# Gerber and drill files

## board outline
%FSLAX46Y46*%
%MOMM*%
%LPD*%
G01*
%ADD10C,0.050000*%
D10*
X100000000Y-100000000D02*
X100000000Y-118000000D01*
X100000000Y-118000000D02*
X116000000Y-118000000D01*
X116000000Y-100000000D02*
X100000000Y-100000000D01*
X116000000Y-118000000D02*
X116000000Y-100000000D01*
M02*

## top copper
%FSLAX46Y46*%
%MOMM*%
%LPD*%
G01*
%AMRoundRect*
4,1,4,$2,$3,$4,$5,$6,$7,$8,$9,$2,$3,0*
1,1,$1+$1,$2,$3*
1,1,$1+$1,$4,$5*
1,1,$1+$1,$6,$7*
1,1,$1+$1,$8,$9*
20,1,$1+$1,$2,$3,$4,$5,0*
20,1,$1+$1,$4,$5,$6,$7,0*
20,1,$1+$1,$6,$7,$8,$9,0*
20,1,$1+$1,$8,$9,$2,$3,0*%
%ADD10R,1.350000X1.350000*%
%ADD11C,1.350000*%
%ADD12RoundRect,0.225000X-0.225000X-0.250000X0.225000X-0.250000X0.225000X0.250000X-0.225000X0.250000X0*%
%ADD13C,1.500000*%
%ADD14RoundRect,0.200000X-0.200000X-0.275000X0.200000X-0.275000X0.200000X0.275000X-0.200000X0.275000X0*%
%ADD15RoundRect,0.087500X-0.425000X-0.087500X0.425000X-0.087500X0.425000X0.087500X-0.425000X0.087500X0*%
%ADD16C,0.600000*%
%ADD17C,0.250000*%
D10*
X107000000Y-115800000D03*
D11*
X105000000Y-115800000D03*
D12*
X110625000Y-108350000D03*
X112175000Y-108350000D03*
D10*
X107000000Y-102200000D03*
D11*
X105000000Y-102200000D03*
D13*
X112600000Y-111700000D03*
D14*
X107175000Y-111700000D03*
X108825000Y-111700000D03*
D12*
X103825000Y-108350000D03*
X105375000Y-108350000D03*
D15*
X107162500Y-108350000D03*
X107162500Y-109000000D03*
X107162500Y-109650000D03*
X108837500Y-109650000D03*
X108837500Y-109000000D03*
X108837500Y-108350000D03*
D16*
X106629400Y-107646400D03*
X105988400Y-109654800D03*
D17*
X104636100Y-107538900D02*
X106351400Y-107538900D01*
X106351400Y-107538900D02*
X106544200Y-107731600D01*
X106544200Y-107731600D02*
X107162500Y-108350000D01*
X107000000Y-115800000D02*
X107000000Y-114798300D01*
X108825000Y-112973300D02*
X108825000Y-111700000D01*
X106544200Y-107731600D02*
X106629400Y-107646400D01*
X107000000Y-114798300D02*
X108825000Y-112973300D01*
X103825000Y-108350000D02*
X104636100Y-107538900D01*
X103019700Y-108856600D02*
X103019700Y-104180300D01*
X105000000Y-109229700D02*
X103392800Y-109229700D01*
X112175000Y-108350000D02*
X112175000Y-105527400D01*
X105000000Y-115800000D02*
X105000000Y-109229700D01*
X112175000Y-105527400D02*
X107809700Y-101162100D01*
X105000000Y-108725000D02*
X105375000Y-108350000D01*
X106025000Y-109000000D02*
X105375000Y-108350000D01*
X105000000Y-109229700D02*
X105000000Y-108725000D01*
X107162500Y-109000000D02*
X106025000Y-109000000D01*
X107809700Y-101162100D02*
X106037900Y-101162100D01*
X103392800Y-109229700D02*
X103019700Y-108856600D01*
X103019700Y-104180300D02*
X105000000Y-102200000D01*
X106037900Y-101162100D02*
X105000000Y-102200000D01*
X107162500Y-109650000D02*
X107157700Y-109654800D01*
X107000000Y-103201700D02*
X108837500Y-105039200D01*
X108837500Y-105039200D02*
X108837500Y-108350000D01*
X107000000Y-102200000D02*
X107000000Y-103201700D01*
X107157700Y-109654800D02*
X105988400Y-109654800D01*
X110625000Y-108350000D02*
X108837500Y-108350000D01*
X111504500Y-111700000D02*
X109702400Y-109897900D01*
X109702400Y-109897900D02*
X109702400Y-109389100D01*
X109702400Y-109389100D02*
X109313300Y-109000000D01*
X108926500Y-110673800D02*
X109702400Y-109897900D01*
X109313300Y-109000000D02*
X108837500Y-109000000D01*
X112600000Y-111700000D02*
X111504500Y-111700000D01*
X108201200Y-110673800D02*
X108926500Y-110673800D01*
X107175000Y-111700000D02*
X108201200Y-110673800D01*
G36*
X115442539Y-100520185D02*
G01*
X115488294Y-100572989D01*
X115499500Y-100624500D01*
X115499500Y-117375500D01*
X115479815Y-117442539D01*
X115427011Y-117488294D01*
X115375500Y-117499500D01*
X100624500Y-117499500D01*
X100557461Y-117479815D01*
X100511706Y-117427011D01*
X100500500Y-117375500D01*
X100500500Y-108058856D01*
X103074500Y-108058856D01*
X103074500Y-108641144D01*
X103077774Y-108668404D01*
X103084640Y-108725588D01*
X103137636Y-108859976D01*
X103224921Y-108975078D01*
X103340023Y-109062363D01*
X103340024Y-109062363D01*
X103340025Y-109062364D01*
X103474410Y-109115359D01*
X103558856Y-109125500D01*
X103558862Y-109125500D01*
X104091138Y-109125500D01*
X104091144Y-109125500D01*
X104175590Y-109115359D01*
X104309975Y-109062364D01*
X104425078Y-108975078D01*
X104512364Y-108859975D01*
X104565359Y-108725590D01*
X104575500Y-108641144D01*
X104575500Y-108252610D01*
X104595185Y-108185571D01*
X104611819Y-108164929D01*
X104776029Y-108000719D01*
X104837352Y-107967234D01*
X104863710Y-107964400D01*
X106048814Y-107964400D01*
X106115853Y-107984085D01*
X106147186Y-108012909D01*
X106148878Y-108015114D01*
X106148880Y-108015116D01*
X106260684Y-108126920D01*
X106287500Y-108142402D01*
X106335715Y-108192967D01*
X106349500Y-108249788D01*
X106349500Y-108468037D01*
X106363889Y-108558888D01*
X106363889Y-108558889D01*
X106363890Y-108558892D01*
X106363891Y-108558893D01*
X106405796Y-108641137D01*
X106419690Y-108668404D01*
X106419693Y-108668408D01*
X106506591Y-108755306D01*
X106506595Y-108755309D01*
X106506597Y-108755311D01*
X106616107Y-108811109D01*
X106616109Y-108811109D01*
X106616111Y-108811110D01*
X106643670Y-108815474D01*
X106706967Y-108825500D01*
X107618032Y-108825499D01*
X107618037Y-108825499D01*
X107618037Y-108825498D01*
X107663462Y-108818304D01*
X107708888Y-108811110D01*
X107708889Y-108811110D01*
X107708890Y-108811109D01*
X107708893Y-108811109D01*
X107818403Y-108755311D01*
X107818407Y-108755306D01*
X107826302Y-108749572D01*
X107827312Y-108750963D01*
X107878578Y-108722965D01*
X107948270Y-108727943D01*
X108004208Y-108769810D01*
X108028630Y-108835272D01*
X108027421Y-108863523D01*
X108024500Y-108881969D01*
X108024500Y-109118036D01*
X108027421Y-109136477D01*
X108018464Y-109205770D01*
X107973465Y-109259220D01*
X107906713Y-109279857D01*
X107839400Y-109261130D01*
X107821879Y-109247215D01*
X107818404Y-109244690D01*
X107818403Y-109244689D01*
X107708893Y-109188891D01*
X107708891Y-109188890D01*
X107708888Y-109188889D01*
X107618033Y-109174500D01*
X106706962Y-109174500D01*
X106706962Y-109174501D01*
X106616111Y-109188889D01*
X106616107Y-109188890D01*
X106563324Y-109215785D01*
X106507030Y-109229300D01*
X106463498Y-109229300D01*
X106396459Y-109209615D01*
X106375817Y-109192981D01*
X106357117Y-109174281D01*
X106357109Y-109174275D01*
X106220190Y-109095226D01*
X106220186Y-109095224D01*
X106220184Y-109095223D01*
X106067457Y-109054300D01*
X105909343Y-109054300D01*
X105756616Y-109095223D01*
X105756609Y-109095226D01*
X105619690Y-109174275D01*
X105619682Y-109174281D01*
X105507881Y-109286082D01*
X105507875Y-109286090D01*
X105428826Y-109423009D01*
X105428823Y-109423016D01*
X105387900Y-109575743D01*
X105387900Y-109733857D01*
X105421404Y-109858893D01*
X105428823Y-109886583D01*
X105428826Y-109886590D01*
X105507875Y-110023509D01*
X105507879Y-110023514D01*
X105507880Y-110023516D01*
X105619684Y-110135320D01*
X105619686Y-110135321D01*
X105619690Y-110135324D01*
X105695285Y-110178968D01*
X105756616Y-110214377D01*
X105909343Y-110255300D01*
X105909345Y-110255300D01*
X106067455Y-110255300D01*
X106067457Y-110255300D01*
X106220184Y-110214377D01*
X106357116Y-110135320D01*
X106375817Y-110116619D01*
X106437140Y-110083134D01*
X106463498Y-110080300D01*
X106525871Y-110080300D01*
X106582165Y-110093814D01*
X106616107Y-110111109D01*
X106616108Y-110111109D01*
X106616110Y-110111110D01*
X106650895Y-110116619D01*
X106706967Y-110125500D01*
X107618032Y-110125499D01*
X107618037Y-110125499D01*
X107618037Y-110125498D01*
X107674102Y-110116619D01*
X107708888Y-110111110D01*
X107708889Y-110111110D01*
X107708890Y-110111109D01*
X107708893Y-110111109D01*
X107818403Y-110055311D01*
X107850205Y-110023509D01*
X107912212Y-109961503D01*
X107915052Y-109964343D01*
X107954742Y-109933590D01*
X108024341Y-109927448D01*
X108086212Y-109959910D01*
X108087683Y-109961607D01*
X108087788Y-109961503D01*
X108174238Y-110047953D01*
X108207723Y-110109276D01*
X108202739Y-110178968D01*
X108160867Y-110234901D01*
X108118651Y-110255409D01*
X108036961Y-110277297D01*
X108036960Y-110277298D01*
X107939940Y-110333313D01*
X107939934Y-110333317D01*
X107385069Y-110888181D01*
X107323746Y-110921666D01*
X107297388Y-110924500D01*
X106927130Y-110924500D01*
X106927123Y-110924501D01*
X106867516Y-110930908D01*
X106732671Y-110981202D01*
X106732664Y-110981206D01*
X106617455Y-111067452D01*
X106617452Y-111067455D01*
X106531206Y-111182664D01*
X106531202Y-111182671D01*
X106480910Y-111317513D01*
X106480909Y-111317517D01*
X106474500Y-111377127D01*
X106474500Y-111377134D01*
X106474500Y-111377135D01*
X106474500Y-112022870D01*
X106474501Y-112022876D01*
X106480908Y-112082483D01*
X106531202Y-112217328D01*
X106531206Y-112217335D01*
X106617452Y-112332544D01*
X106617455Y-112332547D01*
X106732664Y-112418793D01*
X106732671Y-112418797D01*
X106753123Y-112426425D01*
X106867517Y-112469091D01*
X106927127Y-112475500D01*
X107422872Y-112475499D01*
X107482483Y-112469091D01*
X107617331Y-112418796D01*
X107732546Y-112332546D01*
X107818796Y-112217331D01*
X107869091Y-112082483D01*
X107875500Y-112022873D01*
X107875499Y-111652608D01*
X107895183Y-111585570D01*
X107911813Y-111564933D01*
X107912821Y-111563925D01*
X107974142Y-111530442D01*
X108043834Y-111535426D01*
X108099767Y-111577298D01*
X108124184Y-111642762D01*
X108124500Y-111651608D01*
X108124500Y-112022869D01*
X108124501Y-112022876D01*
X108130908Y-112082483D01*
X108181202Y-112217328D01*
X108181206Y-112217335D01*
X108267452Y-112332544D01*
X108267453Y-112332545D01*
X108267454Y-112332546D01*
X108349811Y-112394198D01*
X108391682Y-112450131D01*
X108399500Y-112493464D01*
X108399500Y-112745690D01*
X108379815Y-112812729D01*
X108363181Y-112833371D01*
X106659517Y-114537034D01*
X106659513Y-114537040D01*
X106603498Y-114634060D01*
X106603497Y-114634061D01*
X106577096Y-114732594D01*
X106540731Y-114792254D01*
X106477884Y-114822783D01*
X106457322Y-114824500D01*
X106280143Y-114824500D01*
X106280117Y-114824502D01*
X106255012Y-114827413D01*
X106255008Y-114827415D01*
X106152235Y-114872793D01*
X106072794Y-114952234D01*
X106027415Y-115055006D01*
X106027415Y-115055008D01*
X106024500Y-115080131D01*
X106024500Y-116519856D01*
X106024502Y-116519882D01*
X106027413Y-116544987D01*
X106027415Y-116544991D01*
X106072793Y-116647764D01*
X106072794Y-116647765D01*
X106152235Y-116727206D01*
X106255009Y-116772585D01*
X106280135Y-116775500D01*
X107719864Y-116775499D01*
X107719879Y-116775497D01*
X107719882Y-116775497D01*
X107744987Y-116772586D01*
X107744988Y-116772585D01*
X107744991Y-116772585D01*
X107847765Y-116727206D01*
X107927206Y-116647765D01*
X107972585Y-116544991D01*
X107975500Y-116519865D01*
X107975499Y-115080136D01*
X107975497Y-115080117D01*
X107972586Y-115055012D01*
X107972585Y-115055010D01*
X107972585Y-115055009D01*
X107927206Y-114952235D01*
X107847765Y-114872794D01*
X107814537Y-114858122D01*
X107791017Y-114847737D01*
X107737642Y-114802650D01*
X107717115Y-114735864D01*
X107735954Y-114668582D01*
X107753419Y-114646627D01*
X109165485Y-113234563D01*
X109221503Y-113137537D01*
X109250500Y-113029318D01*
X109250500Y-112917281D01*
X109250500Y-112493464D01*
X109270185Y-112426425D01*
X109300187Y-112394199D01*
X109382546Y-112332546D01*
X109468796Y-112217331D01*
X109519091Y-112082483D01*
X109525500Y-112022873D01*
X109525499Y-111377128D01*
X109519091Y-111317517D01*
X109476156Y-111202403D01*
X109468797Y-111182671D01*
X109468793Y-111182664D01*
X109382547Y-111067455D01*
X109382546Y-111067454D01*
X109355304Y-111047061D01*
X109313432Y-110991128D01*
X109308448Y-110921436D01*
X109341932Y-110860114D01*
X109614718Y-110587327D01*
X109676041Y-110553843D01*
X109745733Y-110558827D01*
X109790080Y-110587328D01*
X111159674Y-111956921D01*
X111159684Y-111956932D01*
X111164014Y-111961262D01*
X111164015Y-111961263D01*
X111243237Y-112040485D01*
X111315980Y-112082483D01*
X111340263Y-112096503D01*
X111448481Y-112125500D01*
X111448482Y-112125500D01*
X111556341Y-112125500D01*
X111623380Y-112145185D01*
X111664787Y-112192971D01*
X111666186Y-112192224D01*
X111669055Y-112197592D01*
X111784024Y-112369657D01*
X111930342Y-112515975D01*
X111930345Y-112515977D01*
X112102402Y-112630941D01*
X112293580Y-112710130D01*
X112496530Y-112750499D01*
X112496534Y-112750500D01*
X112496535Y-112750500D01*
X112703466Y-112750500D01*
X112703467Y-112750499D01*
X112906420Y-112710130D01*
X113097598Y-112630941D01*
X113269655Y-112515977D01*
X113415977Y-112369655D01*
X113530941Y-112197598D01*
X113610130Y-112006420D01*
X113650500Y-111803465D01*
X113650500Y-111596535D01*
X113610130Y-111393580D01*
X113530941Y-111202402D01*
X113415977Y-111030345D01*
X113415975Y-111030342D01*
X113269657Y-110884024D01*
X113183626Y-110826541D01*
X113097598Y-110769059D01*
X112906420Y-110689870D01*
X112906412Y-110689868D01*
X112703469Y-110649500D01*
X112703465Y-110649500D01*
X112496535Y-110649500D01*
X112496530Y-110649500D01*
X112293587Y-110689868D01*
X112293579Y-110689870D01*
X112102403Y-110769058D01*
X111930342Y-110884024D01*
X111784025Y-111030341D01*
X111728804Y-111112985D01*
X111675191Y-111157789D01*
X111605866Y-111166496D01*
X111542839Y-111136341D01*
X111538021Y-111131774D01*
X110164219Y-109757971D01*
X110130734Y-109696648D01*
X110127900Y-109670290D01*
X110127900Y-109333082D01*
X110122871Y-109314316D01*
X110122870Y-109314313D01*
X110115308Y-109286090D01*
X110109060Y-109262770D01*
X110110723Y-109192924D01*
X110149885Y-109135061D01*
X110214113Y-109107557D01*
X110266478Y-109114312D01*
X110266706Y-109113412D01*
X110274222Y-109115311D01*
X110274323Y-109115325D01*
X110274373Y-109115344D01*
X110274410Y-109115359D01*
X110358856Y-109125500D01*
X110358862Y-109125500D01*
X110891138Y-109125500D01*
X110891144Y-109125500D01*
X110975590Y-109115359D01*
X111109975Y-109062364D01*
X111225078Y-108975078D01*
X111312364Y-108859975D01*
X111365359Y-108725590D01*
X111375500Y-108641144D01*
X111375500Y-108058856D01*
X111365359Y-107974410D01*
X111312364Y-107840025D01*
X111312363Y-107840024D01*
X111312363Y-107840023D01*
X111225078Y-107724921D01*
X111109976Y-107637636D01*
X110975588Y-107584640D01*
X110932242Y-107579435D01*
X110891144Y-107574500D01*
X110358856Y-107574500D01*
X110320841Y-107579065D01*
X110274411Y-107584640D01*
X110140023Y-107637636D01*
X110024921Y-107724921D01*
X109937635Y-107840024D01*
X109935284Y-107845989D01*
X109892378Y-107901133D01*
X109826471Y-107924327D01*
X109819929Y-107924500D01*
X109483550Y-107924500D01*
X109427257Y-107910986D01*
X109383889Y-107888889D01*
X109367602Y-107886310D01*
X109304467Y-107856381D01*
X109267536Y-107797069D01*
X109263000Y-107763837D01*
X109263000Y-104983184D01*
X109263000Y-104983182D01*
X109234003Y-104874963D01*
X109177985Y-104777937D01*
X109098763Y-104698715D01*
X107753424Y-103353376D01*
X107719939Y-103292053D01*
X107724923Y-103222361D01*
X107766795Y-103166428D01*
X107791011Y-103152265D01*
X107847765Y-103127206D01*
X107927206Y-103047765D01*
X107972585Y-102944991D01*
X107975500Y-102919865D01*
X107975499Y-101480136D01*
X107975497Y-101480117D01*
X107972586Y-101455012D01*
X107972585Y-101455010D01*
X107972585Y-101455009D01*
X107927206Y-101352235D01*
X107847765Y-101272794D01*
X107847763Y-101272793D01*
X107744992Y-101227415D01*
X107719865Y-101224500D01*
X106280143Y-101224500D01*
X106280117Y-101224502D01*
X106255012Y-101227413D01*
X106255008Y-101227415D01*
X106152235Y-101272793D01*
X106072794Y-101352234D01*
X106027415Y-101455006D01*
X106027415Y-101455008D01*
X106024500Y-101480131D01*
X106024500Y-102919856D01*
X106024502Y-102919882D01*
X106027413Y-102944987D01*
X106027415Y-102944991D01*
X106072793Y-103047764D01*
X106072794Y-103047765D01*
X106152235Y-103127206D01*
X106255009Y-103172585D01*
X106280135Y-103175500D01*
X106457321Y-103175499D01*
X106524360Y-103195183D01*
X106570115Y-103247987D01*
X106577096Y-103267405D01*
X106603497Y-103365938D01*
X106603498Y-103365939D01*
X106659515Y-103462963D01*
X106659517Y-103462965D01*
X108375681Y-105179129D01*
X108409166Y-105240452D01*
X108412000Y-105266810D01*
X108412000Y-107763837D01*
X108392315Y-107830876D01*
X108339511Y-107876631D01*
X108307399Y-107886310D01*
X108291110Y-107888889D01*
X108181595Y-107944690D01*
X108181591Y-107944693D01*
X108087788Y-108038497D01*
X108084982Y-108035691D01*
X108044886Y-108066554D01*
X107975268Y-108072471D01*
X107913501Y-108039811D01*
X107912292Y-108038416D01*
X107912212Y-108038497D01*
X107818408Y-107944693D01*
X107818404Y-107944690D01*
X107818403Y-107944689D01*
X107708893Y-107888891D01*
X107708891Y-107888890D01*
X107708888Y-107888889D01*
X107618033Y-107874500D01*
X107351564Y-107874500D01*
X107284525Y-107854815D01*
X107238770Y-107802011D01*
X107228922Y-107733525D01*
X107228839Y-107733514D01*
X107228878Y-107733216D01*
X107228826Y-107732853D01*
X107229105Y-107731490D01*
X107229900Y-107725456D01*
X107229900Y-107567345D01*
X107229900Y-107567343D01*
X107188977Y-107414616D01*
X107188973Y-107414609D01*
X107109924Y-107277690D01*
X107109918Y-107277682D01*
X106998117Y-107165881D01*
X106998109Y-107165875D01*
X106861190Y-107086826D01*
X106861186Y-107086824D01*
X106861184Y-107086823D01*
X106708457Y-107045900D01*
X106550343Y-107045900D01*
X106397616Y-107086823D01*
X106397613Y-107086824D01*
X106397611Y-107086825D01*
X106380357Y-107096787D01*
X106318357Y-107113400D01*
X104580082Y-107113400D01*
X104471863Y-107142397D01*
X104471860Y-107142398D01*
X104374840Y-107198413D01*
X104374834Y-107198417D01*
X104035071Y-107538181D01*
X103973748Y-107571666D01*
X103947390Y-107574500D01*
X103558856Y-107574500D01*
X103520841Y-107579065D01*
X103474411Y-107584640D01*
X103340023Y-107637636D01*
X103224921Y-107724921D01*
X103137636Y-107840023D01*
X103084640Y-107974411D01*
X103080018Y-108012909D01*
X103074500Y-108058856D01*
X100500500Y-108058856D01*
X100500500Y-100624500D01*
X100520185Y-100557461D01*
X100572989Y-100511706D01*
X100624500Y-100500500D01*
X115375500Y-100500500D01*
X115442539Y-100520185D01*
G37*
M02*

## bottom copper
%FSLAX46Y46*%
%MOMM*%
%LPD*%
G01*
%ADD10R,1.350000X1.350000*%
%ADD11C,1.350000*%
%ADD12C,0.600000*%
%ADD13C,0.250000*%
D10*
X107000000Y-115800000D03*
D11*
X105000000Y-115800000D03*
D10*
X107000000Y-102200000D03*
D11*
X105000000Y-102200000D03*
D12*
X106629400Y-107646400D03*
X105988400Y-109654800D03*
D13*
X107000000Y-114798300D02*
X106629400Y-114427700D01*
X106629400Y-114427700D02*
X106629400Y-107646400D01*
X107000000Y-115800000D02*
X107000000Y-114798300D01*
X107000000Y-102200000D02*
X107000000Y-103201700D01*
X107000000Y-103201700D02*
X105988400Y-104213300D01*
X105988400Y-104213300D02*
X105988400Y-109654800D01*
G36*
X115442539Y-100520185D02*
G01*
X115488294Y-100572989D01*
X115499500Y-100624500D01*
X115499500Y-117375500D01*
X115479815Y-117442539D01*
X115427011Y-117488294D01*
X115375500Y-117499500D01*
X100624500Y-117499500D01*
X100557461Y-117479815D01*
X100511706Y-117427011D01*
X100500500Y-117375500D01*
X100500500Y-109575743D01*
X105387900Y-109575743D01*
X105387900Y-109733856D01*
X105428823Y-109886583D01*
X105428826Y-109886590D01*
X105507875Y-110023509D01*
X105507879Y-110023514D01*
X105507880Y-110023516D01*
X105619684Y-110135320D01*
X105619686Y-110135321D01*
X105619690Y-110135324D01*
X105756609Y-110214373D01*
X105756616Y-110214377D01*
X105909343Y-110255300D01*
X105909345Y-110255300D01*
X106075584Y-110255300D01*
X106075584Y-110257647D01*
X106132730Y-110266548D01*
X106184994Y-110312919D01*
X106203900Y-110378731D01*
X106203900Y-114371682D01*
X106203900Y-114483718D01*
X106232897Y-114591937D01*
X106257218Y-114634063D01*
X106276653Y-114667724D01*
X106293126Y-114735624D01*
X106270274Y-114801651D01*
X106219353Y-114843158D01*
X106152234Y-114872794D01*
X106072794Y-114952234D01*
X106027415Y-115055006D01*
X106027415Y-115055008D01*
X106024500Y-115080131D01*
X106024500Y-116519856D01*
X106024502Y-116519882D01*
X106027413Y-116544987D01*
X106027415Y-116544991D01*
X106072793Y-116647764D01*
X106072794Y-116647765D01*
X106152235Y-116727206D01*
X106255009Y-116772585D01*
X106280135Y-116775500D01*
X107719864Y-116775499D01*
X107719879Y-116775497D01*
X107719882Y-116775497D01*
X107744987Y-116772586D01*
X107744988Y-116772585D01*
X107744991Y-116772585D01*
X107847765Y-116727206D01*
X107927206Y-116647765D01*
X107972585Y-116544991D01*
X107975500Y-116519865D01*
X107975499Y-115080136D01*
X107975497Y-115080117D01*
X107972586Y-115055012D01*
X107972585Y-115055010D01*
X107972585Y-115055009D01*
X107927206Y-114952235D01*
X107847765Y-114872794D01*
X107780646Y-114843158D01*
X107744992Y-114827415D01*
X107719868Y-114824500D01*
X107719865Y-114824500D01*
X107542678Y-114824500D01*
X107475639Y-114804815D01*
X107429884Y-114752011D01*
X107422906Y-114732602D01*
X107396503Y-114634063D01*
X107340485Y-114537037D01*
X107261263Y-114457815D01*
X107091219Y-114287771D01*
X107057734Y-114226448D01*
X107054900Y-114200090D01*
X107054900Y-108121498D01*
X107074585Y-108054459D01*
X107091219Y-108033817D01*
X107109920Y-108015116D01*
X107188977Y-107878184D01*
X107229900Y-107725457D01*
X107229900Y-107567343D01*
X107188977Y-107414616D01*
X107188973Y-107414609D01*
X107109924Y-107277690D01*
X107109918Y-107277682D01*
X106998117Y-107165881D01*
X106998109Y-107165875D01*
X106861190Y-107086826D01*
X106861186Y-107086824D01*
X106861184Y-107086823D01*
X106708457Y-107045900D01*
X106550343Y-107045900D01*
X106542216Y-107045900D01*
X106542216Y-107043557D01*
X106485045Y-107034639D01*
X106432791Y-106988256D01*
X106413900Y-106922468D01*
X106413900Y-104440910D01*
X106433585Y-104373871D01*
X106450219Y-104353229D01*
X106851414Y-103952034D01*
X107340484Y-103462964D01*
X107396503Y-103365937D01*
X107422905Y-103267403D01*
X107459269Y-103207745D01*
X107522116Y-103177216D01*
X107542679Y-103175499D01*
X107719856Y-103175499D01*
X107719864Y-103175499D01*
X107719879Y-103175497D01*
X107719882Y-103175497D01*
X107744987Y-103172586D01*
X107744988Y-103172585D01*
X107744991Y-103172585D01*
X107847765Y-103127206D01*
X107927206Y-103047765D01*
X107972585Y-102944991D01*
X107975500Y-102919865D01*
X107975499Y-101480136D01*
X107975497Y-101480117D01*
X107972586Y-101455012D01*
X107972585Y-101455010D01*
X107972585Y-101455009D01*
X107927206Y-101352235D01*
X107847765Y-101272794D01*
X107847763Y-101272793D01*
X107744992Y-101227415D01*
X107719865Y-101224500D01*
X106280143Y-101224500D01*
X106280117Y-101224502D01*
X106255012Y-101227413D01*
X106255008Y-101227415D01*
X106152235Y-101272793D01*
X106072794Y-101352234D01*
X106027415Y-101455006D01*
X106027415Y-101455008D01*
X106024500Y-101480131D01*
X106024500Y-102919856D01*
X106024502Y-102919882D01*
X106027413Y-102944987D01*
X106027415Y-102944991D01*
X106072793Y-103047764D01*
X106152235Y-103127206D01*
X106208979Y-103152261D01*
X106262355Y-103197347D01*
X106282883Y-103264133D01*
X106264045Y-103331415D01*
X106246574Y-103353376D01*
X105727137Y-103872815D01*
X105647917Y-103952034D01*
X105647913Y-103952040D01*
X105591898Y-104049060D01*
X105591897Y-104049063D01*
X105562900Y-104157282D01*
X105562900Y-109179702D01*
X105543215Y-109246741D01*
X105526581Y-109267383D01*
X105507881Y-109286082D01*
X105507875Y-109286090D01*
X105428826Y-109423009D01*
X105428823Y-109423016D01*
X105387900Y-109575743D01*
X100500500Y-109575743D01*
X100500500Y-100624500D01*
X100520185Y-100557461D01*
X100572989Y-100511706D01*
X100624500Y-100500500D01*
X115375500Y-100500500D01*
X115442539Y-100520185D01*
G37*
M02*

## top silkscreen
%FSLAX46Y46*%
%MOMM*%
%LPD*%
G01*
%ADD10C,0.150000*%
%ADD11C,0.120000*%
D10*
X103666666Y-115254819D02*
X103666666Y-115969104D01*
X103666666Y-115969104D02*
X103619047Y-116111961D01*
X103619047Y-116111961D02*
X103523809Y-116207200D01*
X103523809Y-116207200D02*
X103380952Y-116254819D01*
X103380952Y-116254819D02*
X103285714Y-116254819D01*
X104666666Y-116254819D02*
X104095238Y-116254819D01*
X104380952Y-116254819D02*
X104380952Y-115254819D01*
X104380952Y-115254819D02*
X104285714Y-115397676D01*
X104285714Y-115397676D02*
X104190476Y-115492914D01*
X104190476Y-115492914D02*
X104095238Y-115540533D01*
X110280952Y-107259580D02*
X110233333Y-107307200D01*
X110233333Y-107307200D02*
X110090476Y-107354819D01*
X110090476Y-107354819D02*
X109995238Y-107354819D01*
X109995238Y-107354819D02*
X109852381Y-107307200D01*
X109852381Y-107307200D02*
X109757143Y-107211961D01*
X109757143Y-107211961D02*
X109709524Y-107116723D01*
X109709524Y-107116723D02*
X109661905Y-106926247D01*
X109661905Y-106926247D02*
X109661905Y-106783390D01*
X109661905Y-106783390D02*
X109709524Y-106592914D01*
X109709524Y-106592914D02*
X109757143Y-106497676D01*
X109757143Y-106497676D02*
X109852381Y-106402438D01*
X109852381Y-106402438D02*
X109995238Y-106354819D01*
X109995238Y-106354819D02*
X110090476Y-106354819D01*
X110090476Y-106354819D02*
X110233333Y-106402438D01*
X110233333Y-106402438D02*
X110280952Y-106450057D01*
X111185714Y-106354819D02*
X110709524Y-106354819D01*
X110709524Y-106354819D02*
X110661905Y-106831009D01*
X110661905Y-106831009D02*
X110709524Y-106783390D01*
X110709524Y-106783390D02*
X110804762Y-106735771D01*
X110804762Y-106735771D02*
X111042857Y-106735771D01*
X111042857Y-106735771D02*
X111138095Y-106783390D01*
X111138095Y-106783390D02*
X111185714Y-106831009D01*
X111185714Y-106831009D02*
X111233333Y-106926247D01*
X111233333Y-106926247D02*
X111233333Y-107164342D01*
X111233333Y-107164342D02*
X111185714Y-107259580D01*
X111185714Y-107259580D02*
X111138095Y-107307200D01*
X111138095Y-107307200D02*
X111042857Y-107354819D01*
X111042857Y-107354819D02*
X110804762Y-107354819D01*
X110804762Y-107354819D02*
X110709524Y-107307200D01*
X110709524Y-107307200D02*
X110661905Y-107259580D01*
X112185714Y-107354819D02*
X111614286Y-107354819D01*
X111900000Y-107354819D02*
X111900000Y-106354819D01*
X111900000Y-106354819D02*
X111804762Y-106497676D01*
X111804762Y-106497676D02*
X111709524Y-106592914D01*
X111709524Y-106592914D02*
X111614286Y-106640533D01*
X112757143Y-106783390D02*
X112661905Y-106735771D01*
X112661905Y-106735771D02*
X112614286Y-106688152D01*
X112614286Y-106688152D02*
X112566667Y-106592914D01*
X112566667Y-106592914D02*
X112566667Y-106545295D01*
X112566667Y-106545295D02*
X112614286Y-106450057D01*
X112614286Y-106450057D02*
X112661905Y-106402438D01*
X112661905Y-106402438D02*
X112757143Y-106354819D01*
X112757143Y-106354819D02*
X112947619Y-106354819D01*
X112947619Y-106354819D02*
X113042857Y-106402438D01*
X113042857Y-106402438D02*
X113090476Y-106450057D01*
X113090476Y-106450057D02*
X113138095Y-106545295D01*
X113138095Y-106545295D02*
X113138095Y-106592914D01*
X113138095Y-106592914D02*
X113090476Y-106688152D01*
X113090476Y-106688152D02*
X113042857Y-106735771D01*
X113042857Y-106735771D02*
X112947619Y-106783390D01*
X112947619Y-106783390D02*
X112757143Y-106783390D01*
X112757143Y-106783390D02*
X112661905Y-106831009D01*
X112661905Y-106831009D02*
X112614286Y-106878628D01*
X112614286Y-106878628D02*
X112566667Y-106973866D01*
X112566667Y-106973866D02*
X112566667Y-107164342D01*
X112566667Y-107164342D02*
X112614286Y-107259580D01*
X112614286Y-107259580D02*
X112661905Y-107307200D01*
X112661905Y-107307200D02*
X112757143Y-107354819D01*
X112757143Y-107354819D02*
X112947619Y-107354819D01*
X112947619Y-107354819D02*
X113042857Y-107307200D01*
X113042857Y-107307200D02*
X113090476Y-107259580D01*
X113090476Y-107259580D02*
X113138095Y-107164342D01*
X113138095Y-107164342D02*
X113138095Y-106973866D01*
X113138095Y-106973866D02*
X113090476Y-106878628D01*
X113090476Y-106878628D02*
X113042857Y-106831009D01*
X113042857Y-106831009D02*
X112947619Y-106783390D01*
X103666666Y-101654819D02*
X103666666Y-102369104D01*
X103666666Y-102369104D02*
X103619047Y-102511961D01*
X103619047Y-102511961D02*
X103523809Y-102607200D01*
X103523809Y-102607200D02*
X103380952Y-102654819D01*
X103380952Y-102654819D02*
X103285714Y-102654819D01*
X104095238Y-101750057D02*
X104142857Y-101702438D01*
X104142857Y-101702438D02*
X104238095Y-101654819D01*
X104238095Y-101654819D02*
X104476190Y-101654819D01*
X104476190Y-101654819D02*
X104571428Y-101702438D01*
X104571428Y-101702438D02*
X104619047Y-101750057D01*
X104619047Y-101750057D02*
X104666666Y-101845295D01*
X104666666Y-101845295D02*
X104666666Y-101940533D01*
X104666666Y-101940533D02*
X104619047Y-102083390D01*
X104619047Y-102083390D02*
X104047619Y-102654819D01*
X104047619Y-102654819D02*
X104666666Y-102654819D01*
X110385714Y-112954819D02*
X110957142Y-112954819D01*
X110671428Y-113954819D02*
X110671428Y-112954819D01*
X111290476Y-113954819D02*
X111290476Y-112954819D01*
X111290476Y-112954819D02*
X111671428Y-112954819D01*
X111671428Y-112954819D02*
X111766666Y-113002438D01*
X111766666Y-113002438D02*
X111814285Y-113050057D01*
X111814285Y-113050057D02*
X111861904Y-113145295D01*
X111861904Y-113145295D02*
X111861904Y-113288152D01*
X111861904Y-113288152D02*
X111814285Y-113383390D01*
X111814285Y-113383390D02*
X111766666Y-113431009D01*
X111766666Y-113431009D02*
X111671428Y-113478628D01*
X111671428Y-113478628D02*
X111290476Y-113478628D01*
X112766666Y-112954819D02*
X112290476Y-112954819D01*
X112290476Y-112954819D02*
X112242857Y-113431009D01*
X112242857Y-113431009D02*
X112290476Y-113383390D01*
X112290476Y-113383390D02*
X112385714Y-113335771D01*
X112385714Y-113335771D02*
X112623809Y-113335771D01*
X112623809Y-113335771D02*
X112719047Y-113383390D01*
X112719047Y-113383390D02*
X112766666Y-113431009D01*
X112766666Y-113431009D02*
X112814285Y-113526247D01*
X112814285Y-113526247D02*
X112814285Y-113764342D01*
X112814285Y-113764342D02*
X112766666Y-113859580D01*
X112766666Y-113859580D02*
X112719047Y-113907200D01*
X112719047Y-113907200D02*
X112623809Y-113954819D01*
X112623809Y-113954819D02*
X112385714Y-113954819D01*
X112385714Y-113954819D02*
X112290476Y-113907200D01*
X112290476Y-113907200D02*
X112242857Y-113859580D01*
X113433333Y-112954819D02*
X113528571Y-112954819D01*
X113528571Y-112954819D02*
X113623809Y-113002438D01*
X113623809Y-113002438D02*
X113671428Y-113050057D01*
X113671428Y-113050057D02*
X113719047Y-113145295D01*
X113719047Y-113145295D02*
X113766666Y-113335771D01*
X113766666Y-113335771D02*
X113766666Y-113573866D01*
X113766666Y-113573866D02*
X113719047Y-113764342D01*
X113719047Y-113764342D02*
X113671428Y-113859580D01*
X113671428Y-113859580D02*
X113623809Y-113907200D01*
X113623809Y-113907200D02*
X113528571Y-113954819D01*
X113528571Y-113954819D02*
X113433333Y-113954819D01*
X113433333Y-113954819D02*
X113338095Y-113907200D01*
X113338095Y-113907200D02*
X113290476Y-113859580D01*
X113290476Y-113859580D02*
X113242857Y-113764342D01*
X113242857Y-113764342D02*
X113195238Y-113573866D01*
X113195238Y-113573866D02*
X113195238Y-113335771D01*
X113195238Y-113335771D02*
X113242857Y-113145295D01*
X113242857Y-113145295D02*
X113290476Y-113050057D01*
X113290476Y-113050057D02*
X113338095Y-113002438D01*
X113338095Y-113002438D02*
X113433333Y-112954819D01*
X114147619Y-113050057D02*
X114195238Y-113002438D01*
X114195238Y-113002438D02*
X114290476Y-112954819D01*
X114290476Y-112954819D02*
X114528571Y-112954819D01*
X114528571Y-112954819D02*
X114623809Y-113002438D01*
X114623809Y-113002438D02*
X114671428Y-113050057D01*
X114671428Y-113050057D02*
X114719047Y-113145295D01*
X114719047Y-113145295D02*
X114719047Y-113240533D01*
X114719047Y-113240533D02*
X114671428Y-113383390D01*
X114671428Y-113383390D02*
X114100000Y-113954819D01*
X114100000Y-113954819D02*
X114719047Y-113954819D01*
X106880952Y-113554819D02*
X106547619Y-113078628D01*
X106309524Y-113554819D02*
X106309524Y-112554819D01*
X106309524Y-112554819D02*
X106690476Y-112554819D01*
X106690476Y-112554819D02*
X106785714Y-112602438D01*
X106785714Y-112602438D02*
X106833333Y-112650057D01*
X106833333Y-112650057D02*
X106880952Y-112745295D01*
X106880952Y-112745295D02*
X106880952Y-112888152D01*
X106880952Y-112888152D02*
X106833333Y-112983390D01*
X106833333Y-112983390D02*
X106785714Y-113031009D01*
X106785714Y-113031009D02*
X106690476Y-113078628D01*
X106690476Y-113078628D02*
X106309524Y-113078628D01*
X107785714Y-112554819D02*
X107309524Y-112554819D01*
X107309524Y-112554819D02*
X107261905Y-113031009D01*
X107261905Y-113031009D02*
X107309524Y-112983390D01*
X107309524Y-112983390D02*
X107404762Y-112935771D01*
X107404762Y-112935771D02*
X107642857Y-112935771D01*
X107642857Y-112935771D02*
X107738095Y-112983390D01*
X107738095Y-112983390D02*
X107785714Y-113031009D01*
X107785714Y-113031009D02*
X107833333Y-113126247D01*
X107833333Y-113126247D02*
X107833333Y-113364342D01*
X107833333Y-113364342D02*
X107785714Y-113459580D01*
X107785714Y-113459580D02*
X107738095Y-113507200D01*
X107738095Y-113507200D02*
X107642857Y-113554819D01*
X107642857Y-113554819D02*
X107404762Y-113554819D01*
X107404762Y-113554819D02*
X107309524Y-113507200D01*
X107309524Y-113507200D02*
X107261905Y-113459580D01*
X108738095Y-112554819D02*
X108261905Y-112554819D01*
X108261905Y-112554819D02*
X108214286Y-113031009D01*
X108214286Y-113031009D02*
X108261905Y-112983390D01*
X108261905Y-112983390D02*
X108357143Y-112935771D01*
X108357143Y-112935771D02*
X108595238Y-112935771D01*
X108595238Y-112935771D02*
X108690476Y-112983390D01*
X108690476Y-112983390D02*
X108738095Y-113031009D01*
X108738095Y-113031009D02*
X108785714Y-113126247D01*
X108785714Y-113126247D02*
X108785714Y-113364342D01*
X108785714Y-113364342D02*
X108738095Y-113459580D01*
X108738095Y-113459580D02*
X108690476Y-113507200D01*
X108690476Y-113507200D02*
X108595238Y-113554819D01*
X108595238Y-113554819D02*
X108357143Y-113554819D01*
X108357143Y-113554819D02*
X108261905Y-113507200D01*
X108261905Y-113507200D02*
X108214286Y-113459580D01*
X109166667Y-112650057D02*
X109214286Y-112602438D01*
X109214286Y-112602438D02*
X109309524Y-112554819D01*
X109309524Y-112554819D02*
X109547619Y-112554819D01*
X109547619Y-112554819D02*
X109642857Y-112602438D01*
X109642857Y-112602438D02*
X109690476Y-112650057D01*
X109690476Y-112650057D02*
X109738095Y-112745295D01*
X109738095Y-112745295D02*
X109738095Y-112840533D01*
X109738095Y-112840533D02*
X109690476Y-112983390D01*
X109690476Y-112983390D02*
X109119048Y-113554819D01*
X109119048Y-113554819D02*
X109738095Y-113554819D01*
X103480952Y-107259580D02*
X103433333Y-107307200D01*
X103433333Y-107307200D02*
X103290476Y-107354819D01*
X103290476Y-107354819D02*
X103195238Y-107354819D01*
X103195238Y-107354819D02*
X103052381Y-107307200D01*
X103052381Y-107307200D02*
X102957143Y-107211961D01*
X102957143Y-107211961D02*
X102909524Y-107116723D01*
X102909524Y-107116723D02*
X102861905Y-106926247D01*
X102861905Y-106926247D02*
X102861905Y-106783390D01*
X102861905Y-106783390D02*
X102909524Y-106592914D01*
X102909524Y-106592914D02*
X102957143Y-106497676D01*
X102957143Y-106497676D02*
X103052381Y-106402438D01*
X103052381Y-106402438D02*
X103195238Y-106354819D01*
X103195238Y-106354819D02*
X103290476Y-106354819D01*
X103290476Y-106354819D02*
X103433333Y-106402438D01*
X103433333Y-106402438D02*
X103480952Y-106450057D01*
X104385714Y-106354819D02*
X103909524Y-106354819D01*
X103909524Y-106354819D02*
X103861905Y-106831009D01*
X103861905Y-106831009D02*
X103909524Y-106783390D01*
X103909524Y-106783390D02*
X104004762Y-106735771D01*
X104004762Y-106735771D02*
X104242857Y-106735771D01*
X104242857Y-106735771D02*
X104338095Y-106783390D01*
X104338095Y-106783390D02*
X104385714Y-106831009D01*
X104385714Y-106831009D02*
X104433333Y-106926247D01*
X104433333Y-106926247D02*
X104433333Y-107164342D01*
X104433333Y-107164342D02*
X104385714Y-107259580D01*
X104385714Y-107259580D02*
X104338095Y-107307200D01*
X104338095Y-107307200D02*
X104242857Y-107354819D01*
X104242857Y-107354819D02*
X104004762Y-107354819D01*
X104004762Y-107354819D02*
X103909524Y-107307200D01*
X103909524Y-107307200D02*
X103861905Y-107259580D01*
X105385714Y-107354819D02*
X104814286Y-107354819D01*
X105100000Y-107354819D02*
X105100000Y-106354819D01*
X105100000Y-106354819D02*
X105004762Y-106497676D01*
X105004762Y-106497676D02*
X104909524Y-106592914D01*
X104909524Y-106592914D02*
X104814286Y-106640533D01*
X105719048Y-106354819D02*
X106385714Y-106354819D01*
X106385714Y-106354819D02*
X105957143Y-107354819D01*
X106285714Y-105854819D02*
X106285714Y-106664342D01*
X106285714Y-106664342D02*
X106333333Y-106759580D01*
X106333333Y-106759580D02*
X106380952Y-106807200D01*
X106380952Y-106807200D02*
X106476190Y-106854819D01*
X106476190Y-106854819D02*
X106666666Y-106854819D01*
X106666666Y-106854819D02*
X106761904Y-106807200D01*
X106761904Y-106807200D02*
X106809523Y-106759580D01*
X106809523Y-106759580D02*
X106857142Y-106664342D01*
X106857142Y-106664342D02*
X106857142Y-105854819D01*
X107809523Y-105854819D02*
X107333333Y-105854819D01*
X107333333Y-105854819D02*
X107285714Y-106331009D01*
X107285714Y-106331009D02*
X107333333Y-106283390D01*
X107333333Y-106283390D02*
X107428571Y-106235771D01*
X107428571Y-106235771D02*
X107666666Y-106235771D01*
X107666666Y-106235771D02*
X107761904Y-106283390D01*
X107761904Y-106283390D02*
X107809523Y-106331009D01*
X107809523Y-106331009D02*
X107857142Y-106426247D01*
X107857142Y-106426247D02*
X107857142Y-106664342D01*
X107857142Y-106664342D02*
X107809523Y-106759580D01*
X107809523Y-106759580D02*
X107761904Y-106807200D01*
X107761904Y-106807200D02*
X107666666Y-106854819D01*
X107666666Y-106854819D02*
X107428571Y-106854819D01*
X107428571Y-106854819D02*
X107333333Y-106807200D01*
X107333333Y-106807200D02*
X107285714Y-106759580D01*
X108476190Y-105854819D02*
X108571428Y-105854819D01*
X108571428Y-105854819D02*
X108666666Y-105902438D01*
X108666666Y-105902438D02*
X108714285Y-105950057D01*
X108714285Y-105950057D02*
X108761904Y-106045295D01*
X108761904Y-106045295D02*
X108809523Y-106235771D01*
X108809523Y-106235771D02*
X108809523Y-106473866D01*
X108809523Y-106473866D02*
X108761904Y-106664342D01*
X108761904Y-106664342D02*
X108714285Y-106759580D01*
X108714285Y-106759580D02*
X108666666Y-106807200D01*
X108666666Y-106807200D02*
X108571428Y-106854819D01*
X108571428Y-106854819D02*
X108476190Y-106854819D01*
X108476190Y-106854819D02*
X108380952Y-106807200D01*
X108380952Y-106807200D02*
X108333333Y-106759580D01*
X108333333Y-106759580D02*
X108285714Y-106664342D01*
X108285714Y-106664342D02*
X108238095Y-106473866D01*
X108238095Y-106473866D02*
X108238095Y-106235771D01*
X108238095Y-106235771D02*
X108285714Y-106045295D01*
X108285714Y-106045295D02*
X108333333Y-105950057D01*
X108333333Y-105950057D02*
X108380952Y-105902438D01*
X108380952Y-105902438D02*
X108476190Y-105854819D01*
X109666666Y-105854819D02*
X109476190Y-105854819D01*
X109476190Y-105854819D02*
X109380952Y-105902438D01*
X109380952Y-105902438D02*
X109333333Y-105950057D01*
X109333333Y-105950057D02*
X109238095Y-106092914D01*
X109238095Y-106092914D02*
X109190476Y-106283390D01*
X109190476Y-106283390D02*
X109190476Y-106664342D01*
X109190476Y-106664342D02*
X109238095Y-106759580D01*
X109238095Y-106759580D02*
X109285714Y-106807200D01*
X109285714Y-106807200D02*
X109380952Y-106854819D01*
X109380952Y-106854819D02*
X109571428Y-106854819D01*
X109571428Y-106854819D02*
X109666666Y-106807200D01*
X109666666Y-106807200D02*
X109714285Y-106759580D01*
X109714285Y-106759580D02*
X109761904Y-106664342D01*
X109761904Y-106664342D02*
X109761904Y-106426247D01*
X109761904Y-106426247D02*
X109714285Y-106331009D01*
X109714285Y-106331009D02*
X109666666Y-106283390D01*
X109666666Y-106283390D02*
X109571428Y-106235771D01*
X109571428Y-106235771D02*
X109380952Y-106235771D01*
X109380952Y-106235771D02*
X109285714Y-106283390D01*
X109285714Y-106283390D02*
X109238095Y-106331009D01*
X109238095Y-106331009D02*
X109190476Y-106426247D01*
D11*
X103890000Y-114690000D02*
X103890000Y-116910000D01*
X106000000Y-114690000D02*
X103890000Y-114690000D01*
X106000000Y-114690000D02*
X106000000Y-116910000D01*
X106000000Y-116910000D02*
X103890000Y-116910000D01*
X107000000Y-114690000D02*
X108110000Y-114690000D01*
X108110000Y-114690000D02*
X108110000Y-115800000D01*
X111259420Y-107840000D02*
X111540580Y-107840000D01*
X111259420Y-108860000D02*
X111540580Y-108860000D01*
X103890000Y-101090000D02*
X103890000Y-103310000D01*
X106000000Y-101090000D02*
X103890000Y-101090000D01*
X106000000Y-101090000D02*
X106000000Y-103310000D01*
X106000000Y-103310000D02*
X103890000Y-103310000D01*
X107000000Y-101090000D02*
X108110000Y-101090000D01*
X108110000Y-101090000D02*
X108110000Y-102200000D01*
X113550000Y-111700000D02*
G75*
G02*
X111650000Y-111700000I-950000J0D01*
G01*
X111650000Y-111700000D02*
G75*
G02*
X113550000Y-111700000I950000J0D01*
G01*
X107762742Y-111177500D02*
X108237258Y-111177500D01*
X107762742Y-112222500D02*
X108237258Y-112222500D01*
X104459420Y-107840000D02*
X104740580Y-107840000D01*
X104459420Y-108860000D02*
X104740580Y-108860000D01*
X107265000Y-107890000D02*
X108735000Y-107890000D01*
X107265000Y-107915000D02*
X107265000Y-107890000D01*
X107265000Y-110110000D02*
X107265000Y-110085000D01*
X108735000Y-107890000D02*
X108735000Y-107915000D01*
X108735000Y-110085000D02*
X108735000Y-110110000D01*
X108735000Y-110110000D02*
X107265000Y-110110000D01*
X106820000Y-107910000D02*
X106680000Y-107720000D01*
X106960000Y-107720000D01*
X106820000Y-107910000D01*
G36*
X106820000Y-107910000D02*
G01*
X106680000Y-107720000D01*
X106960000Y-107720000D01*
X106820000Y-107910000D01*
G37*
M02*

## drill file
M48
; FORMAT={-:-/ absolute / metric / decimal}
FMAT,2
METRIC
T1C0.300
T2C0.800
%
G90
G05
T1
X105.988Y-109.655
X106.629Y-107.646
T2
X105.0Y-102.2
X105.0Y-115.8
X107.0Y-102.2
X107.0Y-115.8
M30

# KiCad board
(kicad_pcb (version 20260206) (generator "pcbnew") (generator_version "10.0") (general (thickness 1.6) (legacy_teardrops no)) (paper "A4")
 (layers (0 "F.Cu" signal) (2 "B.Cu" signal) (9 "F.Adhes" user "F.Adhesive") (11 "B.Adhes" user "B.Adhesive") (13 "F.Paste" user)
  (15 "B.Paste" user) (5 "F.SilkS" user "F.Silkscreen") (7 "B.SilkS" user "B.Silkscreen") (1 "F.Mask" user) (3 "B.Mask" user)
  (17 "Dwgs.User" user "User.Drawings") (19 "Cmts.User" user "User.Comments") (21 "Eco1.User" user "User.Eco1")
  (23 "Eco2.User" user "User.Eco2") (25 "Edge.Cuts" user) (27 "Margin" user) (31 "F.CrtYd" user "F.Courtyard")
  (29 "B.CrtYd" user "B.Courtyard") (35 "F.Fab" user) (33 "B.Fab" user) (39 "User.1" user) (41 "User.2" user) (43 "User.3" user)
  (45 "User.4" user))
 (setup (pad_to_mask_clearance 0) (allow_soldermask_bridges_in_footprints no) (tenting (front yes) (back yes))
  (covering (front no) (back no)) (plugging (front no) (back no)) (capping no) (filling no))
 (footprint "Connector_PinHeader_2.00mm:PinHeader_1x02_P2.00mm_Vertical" (layer "F.Cu") (at 107 115.8 -90)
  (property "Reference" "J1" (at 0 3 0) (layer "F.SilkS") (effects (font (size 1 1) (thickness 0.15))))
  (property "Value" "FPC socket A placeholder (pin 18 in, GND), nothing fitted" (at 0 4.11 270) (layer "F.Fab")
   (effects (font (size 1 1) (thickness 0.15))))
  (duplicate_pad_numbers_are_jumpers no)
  (fp_line (start -1.11 3.11) (end 1.11 3.11) (stroke (width 0.12) (type solid)) (layer "F.SilkS"))
  (fp_line (start -1.11 1) (end -1.11 3.11) (stroke (width 0.12) (type solid)) (layer "F.SilkS"))
  (fp_line (start -1.11 1) (end 1.11 1) (stroke (width 0.12) (type solid)) (layer "F.SilkS"))
  (fp_line (start 1.11 1) (end 1.11 3.11) (stroke (width 0.12) (type solid)) (layer "F.SilkS"))
  (fp_line (start -1.11 0) (end -1.11 -1.11) (stroke (width 0.12) (type solid)) (layer "F.SilkS"))
  (fp_line (start -1.11 -1.11) (end 0 -1.11) (stroke (width 0.12) (type solid)) (layer "F.SilkS"))
  (pad "1" thru_hole rect (at 0 0 270) (size 1.35 1.35) (drill 0.8) (layers "*.Cu" "*.Mask") (remove_unused_layers no)
   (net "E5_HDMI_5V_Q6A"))
  (pad "2" thru_hole circle (at 0 2 270) (size 1.35 1.35) (drill 0.8) (layers "*.Cu" "*.Mask") (remove_unused_layers no) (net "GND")))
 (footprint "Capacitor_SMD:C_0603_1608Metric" (layer "F.Cu") (at 111.4 108.35)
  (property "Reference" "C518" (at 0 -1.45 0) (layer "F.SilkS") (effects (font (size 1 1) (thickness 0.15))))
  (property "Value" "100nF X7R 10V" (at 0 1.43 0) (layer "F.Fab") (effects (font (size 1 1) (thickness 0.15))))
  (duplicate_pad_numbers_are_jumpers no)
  (fp_line (start -0.14058 -0.51) (end 0.14058 -0.51) (stroke (width 0.12) (type solid)) (layer "F.SilkS"))
  (fp_line (start -0.14058 0.51) (end 0.14058 0.51) (stroke (width 0.12) (type solid)) (layer "F.SilkS"))
  (pad "1" smd roundrect (at -0.775 0) (size 0.9 0.95) (layers "F.Cu" "F.Mask" "F.Paste") (roundrect_rratio 0.25) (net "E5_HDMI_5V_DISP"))
  (pad "2" smd roundrect (at 0.775 0) (size 0.9 0.95) (layers "F.Cu" "F.Mask" "F.Paste") (roundrect_rratio 0.25) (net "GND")))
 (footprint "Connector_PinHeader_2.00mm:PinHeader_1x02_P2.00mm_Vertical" (layer "F.Cu") (at 107 102.2 -90)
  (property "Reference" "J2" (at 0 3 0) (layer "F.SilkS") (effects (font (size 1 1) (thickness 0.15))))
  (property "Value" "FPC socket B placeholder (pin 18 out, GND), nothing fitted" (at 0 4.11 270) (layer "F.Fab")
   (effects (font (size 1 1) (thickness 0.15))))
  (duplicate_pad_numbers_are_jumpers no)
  (fp_line (start -1.11 3.11) (end 1.11 3.11) (stroke (width 0.12) (type solid)) (layer "F.SilkS"))
  (fp_line (start -1.11 1) (end -1.11 3.11) (stroke (width 0.12) (type solid)) (layer "F.SilkS"))
  (fp_line (start -1.11 1) (end 1.11 1) (stroke (width 0.12) (type solid)) (layer "F.SilkS"))
  (fp_line (start 1.11 1) (end 1.11 3.11) (stroke (width 0.12) (type solid)) (layer "F.SilkS"))
  (fp_line (start -1.11 0) (end -1.11 -1.11) (stroke (width 0.12) (type solid)) (layer "F.SilkS"))
  (fp_line (start -1.11 -1.11) (end 0 -1.11) (stroke (width 0.12) (type solid)) (layer "F.SilkS"))
  (pad "1" thru_hole rect (at 0 0 270) (size 1.35 1.35) (drill 0.8) (layers "*.Cu" "*.Mask") (remove_unused_layers no)
   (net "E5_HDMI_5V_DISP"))
  (pad "2" thru_hole circle (at 0 2 270) (size 1.35 1.35) (drill 0.8) (layers "*.Cu" "*.Mask") (remove_unused_layers no) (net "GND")))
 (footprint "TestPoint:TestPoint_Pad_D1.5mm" (layer "F.Cu") (at 112.6 111.7)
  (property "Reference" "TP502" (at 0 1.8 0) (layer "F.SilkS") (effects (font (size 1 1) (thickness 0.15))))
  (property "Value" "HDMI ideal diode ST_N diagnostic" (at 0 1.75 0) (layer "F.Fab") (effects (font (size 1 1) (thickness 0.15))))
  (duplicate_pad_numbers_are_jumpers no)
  (fp_circle (center 0 0) (end 0 0.95) (stroke (width 0.12) (type solid)) (fill no) (layer "F.SilkS"))
  (pad "1" smd circle (at 0 0) (size 1.5 1.5) (layers "F.Cu" "F.Mask") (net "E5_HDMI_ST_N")))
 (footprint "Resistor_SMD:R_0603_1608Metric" (layer "F.Cu") (at 108 111.7)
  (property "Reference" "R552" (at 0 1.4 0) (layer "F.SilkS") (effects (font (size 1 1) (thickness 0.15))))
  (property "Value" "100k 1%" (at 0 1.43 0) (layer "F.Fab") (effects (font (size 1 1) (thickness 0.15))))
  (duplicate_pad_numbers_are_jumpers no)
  (fp_line (start -0.237258 -0.5225) (end 0.237258 -0.5225) (stroke (width 0.12) (type solid)) (layer "F.SilkS"))
  (fp_line (start -0.237258 0.5225) (end 0.237258 0.5225) (stroke (width 0.12) (type solid)) (layer "F.SilkS"))
  (pad "1" smd roundrect (at -0.825 0) (size 0.8 0.95) (layers "F.Cu" "F.Mask" "F.Paste") (roundrect_rratio 0.25) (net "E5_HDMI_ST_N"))
  (pad "2" smd roundrect (at 0.825 0) (size 0.8 0.95) (layers "F.Cu" "F.Mask" "F.Paste") (roundrect_rratio 0.25) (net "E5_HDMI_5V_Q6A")))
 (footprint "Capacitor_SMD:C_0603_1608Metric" (layer "F.Cu") (at 104.6 108.35)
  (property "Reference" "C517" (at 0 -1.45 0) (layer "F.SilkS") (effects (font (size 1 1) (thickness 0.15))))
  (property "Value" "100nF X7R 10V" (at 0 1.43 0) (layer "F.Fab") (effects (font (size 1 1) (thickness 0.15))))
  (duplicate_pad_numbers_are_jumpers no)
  (fp_line (start -0.14058 -0.51) (end 0.14058 -0.51) (stroke (width 0.12) (type solid)) (layer "F.SilkS"))
  (fp_line (start -0.14058 0.51) (end 0.14058 0.51) (stroke (width 0.12) (type solid)) (layer "F.SilkS"))
  (pad "1" smd roundrect (at -0.775 0) (size 0.9 0.95) (layers "F.Cu" "F.Mask" "F.Paste") (roundrect_rratio 0.25) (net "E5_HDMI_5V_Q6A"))
  (pad "2" smd roundrect (at 0.775 0) (size 0.9 0.95) (layers "F.Cu" "F.Mask" "F.Paste") (roundrect_rratio 0.25) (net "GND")))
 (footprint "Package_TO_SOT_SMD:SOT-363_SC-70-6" (layer "F.Cu") (at 108 109)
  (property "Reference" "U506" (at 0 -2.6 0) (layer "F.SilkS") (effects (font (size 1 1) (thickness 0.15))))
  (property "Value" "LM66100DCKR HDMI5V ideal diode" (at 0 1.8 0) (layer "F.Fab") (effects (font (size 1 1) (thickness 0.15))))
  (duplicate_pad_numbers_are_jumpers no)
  (fp_line (start -0.735 -1.11) (end 0.735 -1.11) (stroke (width 0.12) (type solid)) (layer "F.SilkS"))
  (fp_line (start -0.735 -1.085) (end -0.735 -1.11) (stroke (width 0.12) (type solid)) (layer "F.SilkS"))
  (fp_line (start -0.735 1.11) (end -0.735 1.085) (stroke (width 0.12) (type solid)) (layer "F.SilkS"))
  (fp_line (start 0.735 -1.11) (end 0.735 -1.085) (stroke (width 0.12) (type solid)) (layer "F.SilkS"))
  (fp_line (start 0.735 1.085) (end 0.735 1.11) (stroke (width 0.12) (type solid)) (layer "F.SilkS"))
  (fp_line (start 0.735 1.11) (end -0.735 1.11) (stroke (width 0.12) (type solid)) (layer "F.SilkS"))
  (fp_poly (pts (xy -1.18 -1.09) (xy -1.32 -1.28) (xy -1.04 -1.28)) (stroke (width 0.12) (type solid)) (fill yes) (layer "F.SilkS"))
  (pad "1" smd roundrect (at -0.8375 -0.65) (size 1.025 0.35) (layers "F.Cu" "F.Mask" "F.Paste") (roundrect_rratio 0.25)
   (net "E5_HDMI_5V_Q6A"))
  (pad "2" smd roundrect (at -0.8375 0) (size 1.025 0.35) (layers "F.Cu" "F.Mask" "F.Paste") (roundrect_rratio 0.25) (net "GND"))
  (pad "3" smd roundrect (at -0.8375 0.65) (size 1.025 0.35) (layers "F.Cu" "F.Mask" "F.Paste") (roundrect_rratio 0.25)
   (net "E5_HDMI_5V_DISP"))
  (pad "4" smd roundrect (at 0.8375 0.65) (size 1.025 0.35) (layers "F.Cu" "F.Mask" "F.Paste") (roundrect_rratio 0.25))
  (pad "5" smd roundrect (at 0.8375 0) (size 1.025 0.35) (layers "F.Cu" "F.Mask" "F.Paste") (roundrect_rratio 0.25) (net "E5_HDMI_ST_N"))
  (pad "6" smd roundrect (at 0.8375 -0.65) (size 1.025 0.35) (layers "F.Cu" "F.Mask" "F.Paste") (roundrect_rratio 0.25)
   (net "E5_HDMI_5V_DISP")))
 (gr_line (start 100 100) (end 100 118) (stroke (width 0.05) (type default)) (layer "Edge.Cuts"))
 (gr_line (start 100 118) (end 116 118) (stroke (width 0.05) (type default)) (layer "Edge.Cuts"))
 (gr_line (start 116 100) (end 100 100) (stroke (width 0.05) (type default)) (layer "Edge.Cuts"))
 (gr_line (start 116 118) (end 116 100) (stroke (width 0.05) (type default)) (layer "Edge.Cuts"))
 (segment (start 104.6361 107.5389) (end 106.3514 107.5389) (width 0.25) (layer "F.Cu") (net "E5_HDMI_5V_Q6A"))
 (segment (start 106.3514 107.5389) (end 106.5442 107.7316) (width 0.25) (layer "F.Cu") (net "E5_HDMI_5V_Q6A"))
 (segment (start 106.5442 107.7316) (end 107.1625 108.35) (width 0.25) (layer "F.Cu") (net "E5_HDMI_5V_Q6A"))
 (segment (start 107 115.8) (end 107 114.7983) (width 0.25) (layer "F.Cu") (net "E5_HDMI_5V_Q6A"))
 (segment (start 108.825 112.9733) (end 108.825 111.7) (width 0.25) (layer "F.Cu") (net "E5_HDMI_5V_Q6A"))
 (segment (start 106.5442 107.7316) (end 106.6294 107.6464) (width 0.25) (layer "F.Cu") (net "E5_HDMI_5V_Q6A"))
 (segment (start 107 114.7983) (end 108.825 112.9733) (width 0.25) (layer "F.Cu") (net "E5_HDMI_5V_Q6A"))
 (segment (start 103.825 108.35) (end 104.6361 107.5389) (width 0.25) (layer "F.Cu") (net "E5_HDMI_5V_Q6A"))
 (via (at 106.6294 107.6464) (size 0.6) (drill 0.3) (layers "F.Cu" "B.Cu") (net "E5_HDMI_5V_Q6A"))
 (segment (start 107 114.7983) (end 106.6294 114.4277) (width 0.25) (layer "B.Cu") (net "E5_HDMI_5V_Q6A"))
 (segment (start 106.6294 114.4277) (end 106.6294 107.6464) (width 0.25) (layer "B.Cu") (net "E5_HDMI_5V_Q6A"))
 (segment (start 107 115.8) (end 107 114.7983) (width 0.25) (layer "B.Cu") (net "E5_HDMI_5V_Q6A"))
 (segment (start 103.0197 108.8566) (end 103.0197 104.1803) (width 0.25) (layer "F.Cu") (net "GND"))
 (segment (start 105 109.2297) (end 103.3928 109.2297) (width 0.25) (layer "F.Cu") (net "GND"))
 (segment (start 112.175 108.35) (end 112.175 105.5274) (width 0.25) (layer "F.Cu") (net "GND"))
 (segment (start 105 115.8) (end 105 109.2297) (width 0.25) (layer "F.Cu") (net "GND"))
 (segment (start 112.175 105.5274) (end 107.8097 101.1621) (width 0.25) (layer "F.Cu") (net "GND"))
 (segment (start 105 108.725) (end 105.375 108.35) (width 0.25) (layer "F.Cu") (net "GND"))
 (segment (start 106.025 109) (end 105.375 108.35) (width 0.25) (layer "F.Cu") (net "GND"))
 (segment (start 105 109.2297) (end 105 108.725) (width 0.25) (layer "F.Cu") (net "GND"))
 (segment (start 107.1625 109) (end 106.025 109) (width 0.25) (layer "F.Cu") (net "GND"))
 (segment (start 107.8097 101.1621) (end 106.0379 101.1621) (width 0.25) (layer "F.Cu") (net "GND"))
 (segment (start 103.3928 109.2297) (end 103.0197 108.8566) (width 0.25) (layer "F.Cu") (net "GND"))
 (segment (start 103.0197 104.1803) (end 105 102.2) (width 0.25) (layer "F.Cu") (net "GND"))
 (segment (start 106.0379 101.1621) (end 105 102.2) (width 0.25) (layer "F.Cu") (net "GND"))
 (segment (start 107.1625 109.65) (end 107.1577 109.6548) (width 0.25) (layer "F.Cu") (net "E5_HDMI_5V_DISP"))
 (segment (start 107 103.2017) (end 108.8375 105.0392) (width 0.25) (layer "F.Cu") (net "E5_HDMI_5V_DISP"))
 (segment (start 108.8375 105.0392) (end 108.8375 108.35) (width 0.25) (layer "F.Cu") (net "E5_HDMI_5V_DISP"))
 (segment (start 107 102.2) (end 107 103.2017) (width 0.25) (layer "F.Cu") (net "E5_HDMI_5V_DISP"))
 (segment (start 107.1577 109.6548) (end 105.9884 109.6548) (width 0.25) (layer "F.Cu") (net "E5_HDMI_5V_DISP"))
 (segment (start 110.625 108.35) (end 108.8375 108.35) (width 0.25) (layer "F.Cu") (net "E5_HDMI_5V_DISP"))
 (via (at 105.9884 109.6548) (size 0.6) (drill 0.3) (layers "F.Cu" "B.Cu") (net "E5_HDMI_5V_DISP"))
 (segment (start 107 102.2) (end 107 103.2017) (width 0.25) (layer "B.Cu") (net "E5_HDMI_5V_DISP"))
 (segment (start 107 103.2017) (end 105.9884 104.2133) (width 0.25) (layer "B.Cu") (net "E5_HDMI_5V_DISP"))
 (segment (start 105.9884 104.2133) (end 105.9884 109.6548) (width 0.25) (layer "B.Cu") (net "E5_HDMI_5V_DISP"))
 (segment (start 111.5045 111.7) (end 109.7024 109.8979) (width 0.25) (layer "F.Cu") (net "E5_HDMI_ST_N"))
 (segment (start 109.7024 109.8979) (end 109.7024 109.3891) (width 0.25) (layer "F.Cu") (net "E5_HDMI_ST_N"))
 (segment (start 109.7024 109.3891) (end 109.3133 109) (width 0.25) (layer "F.Cu") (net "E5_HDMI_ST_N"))
 (segment (start 108.9265 110.6738) (end 109.7024 109.8979) (width 0.25) (layer "F.Cu") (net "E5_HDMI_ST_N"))
 (segment (start 109.3133 109) (end 108.8375 109) (width 0.25) (layer "F.Cu") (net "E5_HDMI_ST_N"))
 (segment (start 112.6 111.7) (end 111.5045 111.7) (width 0.25) (layer "F.Cu") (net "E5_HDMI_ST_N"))
 (segment (start 108.2012 110.6738) (end 108.9265 110.6738) (width 0.25) (layer "F.Cu") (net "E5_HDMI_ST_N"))
 (segment (start 107.175 111.7) (end 108.2012 110.6738) (width 0.25) (layer "F.Cu") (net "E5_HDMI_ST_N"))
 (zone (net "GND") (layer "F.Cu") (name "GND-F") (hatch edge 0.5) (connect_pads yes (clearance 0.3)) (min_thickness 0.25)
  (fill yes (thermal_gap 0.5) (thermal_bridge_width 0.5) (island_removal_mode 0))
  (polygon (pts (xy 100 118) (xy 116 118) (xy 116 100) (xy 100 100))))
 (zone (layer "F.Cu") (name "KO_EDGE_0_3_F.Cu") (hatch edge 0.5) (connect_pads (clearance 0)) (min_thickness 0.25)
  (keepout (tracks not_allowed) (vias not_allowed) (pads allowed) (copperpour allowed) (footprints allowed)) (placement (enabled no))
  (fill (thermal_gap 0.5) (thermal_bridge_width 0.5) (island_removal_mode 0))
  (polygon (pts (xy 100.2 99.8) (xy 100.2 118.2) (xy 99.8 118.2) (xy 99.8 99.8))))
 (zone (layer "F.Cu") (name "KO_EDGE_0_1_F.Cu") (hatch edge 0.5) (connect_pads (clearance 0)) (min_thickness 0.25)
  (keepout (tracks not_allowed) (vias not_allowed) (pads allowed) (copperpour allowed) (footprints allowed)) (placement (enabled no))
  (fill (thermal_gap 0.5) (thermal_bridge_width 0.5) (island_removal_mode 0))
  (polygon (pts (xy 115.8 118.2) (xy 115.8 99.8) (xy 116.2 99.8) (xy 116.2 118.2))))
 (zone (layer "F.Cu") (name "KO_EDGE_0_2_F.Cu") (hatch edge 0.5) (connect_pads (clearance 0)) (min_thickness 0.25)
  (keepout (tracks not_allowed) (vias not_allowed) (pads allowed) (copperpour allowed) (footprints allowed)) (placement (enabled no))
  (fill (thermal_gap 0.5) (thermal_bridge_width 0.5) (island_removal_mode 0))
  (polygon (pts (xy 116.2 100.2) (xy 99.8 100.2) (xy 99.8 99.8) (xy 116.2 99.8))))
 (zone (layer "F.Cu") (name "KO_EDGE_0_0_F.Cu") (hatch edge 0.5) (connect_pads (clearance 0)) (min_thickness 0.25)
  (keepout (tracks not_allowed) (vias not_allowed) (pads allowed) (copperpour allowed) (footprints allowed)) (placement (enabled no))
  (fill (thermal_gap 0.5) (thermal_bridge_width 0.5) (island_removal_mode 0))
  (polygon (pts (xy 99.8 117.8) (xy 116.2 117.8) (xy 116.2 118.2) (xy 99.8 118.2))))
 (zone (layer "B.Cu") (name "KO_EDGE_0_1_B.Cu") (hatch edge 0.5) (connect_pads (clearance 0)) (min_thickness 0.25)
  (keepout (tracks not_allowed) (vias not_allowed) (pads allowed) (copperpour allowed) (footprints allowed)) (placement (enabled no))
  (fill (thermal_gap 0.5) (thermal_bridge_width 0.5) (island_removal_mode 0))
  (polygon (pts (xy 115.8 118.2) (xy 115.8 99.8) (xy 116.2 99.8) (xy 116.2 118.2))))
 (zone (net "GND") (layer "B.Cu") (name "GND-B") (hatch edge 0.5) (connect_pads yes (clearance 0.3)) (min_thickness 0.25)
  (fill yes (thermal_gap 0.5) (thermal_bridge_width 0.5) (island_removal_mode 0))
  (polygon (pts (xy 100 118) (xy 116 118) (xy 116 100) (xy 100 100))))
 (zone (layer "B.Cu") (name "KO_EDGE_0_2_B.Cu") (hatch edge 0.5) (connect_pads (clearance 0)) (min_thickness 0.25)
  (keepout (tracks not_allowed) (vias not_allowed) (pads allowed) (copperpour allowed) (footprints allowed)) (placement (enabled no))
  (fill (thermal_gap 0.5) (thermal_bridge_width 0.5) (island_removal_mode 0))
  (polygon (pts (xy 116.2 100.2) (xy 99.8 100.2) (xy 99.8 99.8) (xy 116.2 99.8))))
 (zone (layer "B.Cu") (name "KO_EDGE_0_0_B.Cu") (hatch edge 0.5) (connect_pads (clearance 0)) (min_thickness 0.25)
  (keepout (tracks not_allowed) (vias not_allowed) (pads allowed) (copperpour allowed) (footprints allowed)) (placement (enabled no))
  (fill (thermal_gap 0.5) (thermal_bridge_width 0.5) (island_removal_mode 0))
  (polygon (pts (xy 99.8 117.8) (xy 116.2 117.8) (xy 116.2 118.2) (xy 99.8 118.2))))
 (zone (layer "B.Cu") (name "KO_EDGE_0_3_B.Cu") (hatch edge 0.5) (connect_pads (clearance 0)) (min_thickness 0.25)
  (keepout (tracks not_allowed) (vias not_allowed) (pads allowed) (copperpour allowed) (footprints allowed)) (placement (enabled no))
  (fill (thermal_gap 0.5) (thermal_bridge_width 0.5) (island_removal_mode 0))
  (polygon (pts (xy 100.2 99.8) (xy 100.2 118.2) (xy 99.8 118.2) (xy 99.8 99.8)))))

